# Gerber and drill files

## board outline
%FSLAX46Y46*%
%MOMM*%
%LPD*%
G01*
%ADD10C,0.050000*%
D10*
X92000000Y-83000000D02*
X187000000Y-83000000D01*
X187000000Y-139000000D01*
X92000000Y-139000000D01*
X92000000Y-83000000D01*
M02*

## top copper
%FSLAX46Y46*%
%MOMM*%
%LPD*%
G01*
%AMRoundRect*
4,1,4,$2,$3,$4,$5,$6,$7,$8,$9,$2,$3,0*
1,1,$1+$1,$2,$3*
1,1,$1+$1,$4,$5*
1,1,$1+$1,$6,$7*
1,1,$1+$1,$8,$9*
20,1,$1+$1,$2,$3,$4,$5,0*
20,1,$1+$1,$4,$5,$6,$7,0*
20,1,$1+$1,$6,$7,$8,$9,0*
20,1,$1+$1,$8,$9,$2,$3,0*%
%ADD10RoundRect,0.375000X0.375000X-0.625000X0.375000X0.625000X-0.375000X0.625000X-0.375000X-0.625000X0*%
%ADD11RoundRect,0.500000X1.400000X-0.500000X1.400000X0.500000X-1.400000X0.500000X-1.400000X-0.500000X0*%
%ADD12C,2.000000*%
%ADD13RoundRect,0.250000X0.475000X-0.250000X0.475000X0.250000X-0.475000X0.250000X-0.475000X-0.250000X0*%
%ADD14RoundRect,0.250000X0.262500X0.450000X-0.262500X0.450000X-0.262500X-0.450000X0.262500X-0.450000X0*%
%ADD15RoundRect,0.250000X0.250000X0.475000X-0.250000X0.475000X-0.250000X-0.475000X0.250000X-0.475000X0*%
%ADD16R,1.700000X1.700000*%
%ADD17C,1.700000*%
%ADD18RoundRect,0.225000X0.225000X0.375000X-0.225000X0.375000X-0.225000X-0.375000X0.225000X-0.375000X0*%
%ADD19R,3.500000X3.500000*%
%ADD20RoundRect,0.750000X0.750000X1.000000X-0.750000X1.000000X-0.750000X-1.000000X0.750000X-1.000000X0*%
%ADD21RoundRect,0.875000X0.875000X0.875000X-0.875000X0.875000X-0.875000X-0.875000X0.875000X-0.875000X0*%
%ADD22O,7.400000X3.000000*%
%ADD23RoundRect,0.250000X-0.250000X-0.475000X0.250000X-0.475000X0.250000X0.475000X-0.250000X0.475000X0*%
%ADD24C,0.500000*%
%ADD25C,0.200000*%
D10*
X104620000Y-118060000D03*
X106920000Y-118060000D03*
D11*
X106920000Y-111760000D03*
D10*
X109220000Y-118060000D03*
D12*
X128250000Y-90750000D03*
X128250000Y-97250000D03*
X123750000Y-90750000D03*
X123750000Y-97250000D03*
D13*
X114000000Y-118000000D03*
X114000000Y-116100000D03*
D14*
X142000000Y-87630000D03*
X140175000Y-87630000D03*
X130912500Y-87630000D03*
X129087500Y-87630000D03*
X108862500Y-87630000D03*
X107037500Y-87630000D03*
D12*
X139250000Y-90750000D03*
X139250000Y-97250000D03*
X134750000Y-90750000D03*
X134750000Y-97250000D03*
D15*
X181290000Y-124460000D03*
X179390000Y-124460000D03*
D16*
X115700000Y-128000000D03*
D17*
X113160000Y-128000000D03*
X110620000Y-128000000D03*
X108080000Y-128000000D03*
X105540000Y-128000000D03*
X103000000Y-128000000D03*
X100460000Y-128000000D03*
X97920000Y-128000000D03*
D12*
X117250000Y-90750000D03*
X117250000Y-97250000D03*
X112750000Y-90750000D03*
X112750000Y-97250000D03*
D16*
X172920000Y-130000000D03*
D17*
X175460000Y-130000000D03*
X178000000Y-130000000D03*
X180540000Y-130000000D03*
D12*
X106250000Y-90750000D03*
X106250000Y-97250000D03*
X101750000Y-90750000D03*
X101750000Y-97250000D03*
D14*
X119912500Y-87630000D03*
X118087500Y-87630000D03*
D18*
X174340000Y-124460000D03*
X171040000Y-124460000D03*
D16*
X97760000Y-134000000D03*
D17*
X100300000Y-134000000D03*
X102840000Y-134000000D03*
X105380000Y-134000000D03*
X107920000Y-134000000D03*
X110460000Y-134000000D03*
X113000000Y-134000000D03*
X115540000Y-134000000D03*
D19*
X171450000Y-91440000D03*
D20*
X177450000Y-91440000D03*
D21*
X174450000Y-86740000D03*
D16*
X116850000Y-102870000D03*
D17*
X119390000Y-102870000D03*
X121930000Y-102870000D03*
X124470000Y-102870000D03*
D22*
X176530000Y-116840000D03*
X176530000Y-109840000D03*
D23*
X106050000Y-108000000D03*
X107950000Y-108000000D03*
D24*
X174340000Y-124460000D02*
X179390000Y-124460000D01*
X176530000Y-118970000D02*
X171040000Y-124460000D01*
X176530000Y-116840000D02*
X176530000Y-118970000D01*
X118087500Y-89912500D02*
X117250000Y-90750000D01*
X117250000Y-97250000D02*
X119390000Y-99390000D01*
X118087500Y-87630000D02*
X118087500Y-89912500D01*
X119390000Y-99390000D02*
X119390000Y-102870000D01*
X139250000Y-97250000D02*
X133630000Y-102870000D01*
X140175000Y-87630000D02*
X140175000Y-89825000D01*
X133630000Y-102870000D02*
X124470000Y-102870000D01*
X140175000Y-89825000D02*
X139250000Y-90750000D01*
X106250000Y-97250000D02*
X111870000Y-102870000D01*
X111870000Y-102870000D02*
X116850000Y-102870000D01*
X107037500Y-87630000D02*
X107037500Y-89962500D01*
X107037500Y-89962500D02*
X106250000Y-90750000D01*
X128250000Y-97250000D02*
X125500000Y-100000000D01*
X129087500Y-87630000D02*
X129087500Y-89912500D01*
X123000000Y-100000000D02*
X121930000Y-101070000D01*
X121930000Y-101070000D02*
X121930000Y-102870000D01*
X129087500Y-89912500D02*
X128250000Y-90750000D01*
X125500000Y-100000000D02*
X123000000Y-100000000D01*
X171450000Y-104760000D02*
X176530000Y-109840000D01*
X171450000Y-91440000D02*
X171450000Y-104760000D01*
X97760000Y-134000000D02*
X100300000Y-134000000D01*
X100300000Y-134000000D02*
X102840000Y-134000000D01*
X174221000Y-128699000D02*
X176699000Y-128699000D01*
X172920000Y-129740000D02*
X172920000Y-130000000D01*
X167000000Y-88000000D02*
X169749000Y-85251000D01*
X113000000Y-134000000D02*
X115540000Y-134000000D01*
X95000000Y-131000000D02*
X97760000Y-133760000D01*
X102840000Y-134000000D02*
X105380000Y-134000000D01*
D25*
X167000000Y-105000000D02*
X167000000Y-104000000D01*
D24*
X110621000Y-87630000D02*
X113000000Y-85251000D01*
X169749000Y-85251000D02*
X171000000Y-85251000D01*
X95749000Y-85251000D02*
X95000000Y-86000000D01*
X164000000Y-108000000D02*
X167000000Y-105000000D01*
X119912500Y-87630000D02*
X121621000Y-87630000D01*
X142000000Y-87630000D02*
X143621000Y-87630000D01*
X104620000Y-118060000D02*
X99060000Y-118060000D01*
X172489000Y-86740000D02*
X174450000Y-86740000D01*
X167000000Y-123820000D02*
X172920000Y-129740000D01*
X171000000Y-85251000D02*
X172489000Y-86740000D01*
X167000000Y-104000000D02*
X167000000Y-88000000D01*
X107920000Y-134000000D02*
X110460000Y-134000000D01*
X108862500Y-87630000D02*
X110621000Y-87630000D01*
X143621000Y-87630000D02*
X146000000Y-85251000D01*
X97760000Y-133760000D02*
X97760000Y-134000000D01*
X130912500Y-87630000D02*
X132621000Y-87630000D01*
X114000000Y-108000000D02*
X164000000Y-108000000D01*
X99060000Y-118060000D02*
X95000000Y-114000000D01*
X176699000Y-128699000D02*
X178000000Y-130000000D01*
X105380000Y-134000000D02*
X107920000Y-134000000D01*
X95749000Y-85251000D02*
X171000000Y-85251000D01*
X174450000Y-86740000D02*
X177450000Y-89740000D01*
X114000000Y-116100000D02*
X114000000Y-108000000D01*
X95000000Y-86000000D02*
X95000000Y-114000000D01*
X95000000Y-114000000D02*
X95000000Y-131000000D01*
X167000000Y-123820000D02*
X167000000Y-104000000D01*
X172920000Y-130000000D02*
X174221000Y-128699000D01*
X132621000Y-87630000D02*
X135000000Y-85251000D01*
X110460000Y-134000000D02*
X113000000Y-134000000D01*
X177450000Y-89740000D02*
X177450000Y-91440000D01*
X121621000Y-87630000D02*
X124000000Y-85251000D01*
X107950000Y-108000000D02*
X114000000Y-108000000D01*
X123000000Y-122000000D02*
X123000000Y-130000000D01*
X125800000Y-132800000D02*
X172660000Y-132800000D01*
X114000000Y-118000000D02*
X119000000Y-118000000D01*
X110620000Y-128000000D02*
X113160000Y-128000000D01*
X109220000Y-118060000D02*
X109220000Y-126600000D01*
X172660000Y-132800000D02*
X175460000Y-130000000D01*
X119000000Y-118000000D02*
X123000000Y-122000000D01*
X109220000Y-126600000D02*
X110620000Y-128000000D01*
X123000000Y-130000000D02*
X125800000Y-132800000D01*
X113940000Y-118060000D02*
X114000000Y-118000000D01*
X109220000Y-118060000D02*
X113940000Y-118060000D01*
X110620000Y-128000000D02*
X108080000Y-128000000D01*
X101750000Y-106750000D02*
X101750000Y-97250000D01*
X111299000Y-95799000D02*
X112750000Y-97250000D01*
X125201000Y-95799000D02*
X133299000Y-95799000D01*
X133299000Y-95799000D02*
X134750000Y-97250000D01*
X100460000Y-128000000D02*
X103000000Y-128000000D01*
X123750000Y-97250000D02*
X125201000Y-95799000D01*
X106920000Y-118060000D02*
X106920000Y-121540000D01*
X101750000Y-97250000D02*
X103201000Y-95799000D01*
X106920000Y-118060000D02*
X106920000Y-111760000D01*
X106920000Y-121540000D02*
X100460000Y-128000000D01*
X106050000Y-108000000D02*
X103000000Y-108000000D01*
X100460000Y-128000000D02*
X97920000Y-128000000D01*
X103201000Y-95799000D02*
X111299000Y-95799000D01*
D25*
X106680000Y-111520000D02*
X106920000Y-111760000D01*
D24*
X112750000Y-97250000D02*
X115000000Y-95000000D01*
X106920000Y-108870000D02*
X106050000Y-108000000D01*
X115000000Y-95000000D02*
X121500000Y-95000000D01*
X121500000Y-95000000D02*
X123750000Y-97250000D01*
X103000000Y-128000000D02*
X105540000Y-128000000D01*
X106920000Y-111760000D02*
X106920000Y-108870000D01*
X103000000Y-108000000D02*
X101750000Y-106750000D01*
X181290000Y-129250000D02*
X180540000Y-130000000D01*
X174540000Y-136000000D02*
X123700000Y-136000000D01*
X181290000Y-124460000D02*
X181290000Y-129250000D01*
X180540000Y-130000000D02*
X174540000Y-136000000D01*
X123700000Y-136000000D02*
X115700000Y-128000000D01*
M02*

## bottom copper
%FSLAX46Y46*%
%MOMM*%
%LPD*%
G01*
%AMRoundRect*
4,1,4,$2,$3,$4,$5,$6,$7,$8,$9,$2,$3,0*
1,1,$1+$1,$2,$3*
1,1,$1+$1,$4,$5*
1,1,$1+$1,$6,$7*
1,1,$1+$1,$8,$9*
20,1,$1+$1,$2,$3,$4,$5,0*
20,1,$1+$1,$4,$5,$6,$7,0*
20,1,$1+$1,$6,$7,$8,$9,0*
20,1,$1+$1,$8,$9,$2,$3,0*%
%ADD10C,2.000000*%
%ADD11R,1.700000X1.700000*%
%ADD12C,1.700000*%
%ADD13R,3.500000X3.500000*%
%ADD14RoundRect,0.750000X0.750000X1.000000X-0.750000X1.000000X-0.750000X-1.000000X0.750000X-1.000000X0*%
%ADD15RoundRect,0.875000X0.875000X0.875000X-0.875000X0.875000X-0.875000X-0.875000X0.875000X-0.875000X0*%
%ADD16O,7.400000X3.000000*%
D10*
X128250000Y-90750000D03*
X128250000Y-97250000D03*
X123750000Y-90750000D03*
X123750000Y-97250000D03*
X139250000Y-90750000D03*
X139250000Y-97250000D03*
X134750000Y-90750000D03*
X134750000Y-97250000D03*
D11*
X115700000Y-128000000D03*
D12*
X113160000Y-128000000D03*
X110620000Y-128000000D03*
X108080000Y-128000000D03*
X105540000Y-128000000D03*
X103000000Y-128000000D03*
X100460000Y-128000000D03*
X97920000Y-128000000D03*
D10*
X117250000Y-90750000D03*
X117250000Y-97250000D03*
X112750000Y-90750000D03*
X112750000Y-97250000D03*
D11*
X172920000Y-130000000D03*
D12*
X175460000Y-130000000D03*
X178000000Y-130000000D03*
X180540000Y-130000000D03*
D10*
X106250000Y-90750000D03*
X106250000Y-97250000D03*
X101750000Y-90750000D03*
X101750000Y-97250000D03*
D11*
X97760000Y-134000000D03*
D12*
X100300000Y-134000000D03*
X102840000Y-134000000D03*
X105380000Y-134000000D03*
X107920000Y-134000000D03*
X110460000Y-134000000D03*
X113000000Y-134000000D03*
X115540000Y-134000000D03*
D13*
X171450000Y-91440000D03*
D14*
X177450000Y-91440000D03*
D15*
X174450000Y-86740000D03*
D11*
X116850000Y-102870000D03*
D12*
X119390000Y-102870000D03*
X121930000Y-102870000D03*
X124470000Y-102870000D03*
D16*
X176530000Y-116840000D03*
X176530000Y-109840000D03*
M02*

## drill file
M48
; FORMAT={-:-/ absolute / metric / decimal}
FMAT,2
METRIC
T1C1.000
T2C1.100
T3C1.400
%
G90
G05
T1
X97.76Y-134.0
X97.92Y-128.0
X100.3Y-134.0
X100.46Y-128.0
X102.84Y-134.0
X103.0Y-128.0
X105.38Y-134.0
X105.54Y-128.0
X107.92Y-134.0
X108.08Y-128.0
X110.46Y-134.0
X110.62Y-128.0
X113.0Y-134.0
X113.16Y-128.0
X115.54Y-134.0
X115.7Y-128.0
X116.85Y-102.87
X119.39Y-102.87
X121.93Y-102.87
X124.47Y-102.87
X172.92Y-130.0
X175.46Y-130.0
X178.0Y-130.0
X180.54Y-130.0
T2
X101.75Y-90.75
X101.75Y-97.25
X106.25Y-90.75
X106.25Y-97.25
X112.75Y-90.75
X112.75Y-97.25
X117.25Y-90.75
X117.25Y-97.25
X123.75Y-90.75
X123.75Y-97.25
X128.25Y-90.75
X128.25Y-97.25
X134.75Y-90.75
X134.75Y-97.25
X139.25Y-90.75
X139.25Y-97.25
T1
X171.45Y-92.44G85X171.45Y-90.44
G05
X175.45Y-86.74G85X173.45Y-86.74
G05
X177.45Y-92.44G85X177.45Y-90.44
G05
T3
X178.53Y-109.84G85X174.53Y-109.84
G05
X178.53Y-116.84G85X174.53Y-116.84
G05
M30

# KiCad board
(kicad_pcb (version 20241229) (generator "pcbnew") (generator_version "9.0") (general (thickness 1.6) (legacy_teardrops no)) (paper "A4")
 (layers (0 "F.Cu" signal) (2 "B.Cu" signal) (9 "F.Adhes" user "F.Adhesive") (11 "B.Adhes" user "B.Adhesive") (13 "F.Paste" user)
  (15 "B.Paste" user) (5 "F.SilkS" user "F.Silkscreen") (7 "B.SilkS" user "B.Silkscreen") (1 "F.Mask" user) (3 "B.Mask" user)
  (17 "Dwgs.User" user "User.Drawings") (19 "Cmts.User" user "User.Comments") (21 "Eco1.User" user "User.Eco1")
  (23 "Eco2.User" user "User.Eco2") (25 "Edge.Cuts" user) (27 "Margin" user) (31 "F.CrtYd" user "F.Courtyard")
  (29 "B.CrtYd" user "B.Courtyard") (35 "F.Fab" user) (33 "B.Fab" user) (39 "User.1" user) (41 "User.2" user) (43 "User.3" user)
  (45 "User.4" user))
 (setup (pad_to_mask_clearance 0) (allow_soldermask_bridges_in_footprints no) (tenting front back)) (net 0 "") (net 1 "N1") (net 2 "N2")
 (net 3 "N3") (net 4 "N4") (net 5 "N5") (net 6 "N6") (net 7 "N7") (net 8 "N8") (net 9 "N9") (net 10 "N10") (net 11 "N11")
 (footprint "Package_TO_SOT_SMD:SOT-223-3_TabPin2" (layer "F.Cu") (at 106.92 114.91 90)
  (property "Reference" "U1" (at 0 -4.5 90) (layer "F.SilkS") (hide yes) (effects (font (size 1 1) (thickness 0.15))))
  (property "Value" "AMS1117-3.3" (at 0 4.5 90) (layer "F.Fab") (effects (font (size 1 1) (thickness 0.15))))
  (pad "1" smd roundrect (at -3.15 -2.3 90) (size 2 1.5) (layers "F.Cu" "F.Mask" "F.Paste") (roundrect_rratio 0.25) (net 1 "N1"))
  (pad "2" smd roundrect (at -3.15 0 90) (size 2 1.5) (layers "F.Cu" "F.Mask" "F.Paste") (roundrect_rratio 0.25) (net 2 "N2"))
  (pad "2" smd roundrect (at 3.15 0 90) (size 2 3.8) (layers "F.Cu" "F.Mask" "F.Paste") (roundrect_rratio 0.25) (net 2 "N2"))
  (pad "3" smd roundrect (at -3.15 2.3 90) (size 2 1.5) (layers "F.Cu" "F.Mask" "F.Paste") (roundrect_rratio 0.25) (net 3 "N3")))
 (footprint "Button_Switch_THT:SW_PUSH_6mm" (layer "F.Cu") (at 128.25 90.75 -90)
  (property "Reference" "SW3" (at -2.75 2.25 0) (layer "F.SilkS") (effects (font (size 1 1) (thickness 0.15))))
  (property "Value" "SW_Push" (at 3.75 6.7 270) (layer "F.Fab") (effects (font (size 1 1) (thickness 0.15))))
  (pad "1" thru_hole circle (at 0 0) (size 2 2) (drill 1.1) (layers "*.Cu" "*.Mask") (remove_unused_layers no) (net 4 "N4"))
  (pad "1" thru_hole circle (at 6.5 0) (size 2 2) (drill 1.1) (layers "*.Cu" "*.Mask") (remove_unused_layers no) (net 4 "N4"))
  (pad "2" thru_hole circle (at 0 4.5) (size 2 2) (drill 1.1) (layers "*.Cu" "*.Mask") (remove_unused_layers no) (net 2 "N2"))
  (pad "2" thru_hole circle (at 6.5 4.5) (size 2 2) (drill 1.1) (layers "*.Cu" "*.Mask") (remove_unused_layers no) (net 2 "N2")))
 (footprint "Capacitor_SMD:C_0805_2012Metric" (layer "F.Cu") (at 114 117.05 90)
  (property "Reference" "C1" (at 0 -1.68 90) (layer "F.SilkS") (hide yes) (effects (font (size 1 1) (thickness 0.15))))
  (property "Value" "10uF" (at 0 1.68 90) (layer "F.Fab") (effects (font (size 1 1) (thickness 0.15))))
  (pad "1" smd roundrect (at -0.95 0 90) (size 1 1.45) (layers "F.Cu" "F.Mask" "F.Paste") (roundrect_rratio 0.25) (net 3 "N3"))
  (pad "2" smd roundrect (at 0.95 0 90) (size 1 1.45) (layers "F.Cu" "F.Mask" "F.Paste") (roundrect_rratio 0.25) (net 1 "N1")))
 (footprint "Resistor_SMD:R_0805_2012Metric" (layer "F.Cu") (at 141.0875 87.63 180)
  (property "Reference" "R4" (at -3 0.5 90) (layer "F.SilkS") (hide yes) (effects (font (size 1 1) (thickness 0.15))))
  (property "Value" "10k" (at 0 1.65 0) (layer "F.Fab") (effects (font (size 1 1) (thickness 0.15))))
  (pad "1" smd roundrect (at -0.9125 0 180) (size 1.025 1.4) (layers "F.Cu" "F.Mask" "F.Paste") (roundrect_rratio 0.243902) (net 1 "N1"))
  (pad "2" smd roundrect (at 0.9125 0 180) (size 1.025 1.4) (layers "F.Cu" "F.Mask" "F.Paste") (roundrect_rratio 0.243902) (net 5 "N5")))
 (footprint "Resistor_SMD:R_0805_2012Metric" (layer "F.Cu") (at 130 87.63 180)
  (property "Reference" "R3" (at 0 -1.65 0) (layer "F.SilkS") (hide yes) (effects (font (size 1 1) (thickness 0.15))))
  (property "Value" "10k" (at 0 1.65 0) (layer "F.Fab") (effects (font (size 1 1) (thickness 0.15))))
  (pad "1" smd roundrect (at -0.9125 0 180) (size 1.025 1.4) (layers "F.Cu" "F.Mask" "F.Paste") (roundrect_rratio 0.243902) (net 1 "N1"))
  (pad "2" smd roundrect (at 0.9125 0 180) (size 1.025 1.4) (layers "F.Cu" "F.Mask" "F.Paste") (roundrect_rratio 0.243902) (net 4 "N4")))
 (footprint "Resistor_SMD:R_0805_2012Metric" (layer "F.Cu") (at 107.95 87.63 180)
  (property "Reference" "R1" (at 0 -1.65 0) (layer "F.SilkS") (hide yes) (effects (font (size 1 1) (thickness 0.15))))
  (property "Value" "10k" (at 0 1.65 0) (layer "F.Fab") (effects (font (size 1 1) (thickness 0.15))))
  (pad "1" smd roundrect (at -0.9125 0 180) (size 1.025 1.4) (layers "F.Cu" "F.Mask" "F.Paste") (roundrect_rratio 0.243902) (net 1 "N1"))
  (pad "2" smd roundrect (at 0.9125 0 180) (size 1.025 1.4) (layers "F.Cu" "F.Mask" "F.Paste") (roundrect_rratio 0.243902) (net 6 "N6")))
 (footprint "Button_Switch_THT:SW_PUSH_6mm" (layer "F.Cu") (at 139.25 90.75 -90)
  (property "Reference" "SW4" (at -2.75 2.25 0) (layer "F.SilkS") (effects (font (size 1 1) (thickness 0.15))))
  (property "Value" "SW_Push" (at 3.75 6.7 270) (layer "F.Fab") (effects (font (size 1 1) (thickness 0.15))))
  (pad "1" thru_hole circle (at 0 0) (size 2 2) (drill 1.1) (layers "*.Cu" "*.Mask") (remove_unused_layers no) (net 5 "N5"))
  (pad "1" thru_hole circle (at 6.5 0) (size 2 2) (drill 1.1) (layers "*.Cu" "*.Mask") (remove_unused_layers no) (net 5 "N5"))
  (pad "2" thru_hole circle (at 0 4.5) (size 2 2) (drill 1.1) (layers "*.Cu" "*.Mask") (remove_unused_layers no) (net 2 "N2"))
  (pad "2" thru_hole circle (at 6.5 4.5) (size 2 2) (drill 1.1) (layers "*.Cu" "*.Mask") (remove_unused_layers no) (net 2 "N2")))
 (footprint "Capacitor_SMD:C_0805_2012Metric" (layer "F.Cu") (at 180.34 124.46 180)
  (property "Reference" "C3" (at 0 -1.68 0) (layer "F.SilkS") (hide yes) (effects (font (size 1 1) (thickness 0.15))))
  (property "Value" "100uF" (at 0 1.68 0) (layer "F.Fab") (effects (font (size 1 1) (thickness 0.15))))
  (pad "1" smd roundrect (at -0.95 0 180) (size 1 1.45) (layers "F.Cu" "F.Mask" "F.Paste") (roundrect_rratio 0.25) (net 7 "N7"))
  (pad "2" smd roundrect (at 0.95 0 180) (size 1 1.45) (layers "F.Cu" "F.Mask" "F.Paste") (roundrect_rratio 0.25) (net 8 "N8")))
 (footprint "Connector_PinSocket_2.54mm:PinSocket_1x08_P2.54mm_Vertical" (layer "F.Cu") (at 115.7 128 -90)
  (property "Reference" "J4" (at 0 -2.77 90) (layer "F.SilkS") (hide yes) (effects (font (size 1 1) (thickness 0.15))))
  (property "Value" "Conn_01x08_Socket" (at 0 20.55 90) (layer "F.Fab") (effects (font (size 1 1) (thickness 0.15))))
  (pad "1" thru_hole rect (at 0 0 270) (size 1.7 1.7) (drill 1) (layers "*.Cu" "*.Mask") (remove_unused_layers no) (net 7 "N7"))
  (pad "2" thru_hole circle (at 0 2.54 270) (size 1.7 1.7) (drill 1) (layers "*.Cu" "*.Mask") (remove_unused_layers no) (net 3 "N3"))
  (pad "3" thru_hole circle (at 0 5.08 270) (size 1.7 1.7) (drill 1) (layers "*.Cu" "*.Mask") (remove_unused_layers no) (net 3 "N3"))
  (pad "4" thru_hole circle (at 0 7.62 270) (size 1.7 1.7) (drill 1) (layers "*.Cu" "*.Mask") (remove_unused_layers no) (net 3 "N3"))
  (pad "5" thru_hole circle (at 0 10.16 270) (size 1.7 1.7) (drill 1) (layers "*.Cu" "*.Mask") (remove_unused_layers no) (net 2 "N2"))
  (pad "6" thru_hole circle (at 0 12.7 270) (size 1.7 1.7) (drill 1) (layers "*.Cu" "*.Mask") (remove_unused_layers no) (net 2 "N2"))
  (pad "7" thru_hole circle (at 0 15.24 270) (size 1.7 1.7) (drill 1) (layers "*.Cu" "*.Mask") (remove_unused_layers no) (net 2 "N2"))
  (pad "8" thru_hole circle (at 0 17.78 270) (size 1.7 1.7) (drill 1) (layers "*.Cu" "*.Mask") (remove_unused_layers no) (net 2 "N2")))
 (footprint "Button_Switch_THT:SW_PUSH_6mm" (layer "F.Cu") (at 117.25 90.75 -90)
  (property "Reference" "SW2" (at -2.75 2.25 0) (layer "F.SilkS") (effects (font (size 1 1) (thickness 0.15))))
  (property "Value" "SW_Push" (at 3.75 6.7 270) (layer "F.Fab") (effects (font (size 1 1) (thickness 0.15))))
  (pad "1" thru_hole circle (at 0 0) (size 2 2) (drill 1.1) (layers "*.Cu" "*.Mask") (remove_unused_layers no) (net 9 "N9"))
  (pad "1" thru_hole circle (at 6.5 0) (size 2 2) (drill 1.1) (layers "*.Cu" "*.Mask") (remove_unused_layers no) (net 9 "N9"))
  (pad "2" thru_hole circle (at 0 4.5) (size 2 2) (drill 1.1) (layers "*.Cu" "*.Mask") (remove_unused_layers no) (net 2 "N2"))
  (pad "2" thru_hole circle (at 6.5 4.5) (size 2 2) (drill 1.1) (layers "*.Cu" "*.Mask") (remove_unused_layers no) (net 2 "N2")))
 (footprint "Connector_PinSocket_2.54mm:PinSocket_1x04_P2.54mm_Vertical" (layer "F.Cu") (at 172.92 130 90)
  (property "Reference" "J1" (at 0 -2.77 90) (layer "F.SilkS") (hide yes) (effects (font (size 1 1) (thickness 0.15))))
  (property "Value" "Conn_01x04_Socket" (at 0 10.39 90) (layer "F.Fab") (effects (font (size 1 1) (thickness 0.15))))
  (pad "1" thru_hole rect (at 0 0 90) (size 1.7 1.7) (drill 1) (layers "*.Cu" "*.Mask") (remove_unused_layers no) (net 1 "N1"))
  (pad "2" thru_hole circle (at 0 2.54 90) (size 1.7 1.7) (drill 1) (layers "*.Cu" "*.Mask") (remove_unused_layers no) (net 3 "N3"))
  (pad "3" thru_hole circle (at 0 5.08 90) (size 1.7 1.7) (drill 1) (layers "*.Cu" "*.Mask") (remove_unused_layers no) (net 1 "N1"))
  (pad "4" thru_hole circle (at 0 7.62 90) (size 1.7 1.7) (drill 1) (layers "*.Cu" "*.Mask") (remove_unused_layers no) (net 7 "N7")))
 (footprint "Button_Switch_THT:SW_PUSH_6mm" (layer "F.Cu") (at 106.25 90.75 -90)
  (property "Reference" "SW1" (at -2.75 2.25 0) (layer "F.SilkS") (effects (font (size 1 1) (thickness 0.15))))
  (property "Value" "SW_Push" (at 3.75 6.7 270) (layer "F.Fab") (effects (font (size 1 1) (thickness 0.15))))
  (pad "1" thru_hole circle (at 0 0) (size 2 2) (drill 1.1) (layers "*.Cu" "*.Mask") (remove_unused_layers no) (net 6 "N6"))
  (pad "1" thru_hole circle (at 6.5 0) (size 2 2) (drill 1.1) (layers "*.Cu" "*.Mask") (remove_unused_layers no) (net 6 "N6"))
  (pad "2" thru_hole circle (at 0 4.5) (size 2 2) (drill 1.1) (layers "*.Cu" "*.Mask") (remove_unused_layers no) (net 2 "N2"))
  (pad "2" thru_hole circle (at 6.5 4.5) (size 2 2) (drill 1.1) (layers "*.Cu" "*.Mask") (remove_unused_layers no) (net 2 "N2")))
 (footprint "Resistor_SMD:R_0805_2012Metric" (layer "F.Cu") (at 119 87.63 180)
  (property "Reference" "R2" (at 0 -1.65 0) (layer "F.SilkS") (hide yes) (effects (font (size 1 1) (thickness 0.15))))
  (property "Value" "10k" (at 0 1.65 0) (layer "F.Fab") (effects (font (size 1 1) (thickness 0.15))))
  (pad "1" smd roundrect (at -0.9125 0 180) (size 1.025 1.4) (layers "F.Cu" "F.Mask" "F.Paste") (roundrect_rratio 0.243902) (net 1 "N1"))
  (pad "2" smd roundrect (at 0.9125 0 180) (size 1.025 1.4) (layers "F.Cu" "F.Mask" "F.Paste") (roundrect_rratio 0.243902) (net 9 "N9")))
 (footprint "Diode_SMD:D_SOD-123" (layer "F.Cu") (at 172.69 124.46 180)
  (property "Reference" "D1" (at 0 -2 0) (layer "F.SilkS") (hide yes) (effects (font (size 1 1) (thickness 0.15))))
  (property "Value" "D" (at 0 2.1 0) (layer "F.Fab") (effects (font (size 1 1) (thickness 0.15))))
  (pad "1" smd roundrect (at -1.65 0 180) (size 0.9 1.2) (layers "F.Cu" "F.Mask" "F.Paste") (roundrect_rratio 0.25) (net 8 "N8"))
  (pad "2" smd roundrect (at 1.65 0 180) (size 0.9 1.2) (layers "F.Cu" "F.Mask" "F.Paste") (roundrect_rratio 0.25) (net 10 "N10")))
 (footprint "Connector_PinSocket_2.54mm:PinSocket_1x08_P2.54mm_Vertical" (layer "F.Cu") (at 97.76 134 90)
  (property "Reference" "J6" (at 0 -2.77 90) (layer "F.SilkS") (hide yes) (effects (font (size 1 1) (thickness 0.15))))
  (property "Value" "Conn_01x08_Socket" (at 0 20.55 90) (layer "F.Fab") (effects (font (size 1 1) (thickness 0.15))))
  (pad "1" thru_hole rect (at 0 0 90) (size 1.7 1.7) (drill 1) (layers "*.Cu" "*.Mask") (remove_unused_layers no) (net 1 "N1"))
  (pad "2" thru_hole circle (at 0 2.54 90) (size 1.7 1.7) (drill 1) (layers "*.Cu" "*.Mask") (remove_unused_layers no) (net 1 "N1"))
  (pad "3" thru_hole circle (at 0 5.08 90) (size 1.7 1.7) (drill 1) (layers "*.Cu" "*.Mask") (remove_unused_layers no) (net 1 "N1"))
  (pad "4" thru_hole circle (at 0 7.62 90) (size 1.7 1.7) (drill 1) (layers "*.Cu" "*.Mask") (remove_unused_layers no) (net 1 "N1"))
  (pad "5" thru_hole circle (at 0 10.16 90) (size 1.7 1.7) (drill 1) (layers "*.Cu" "*.Mask") (remove_unused_layers no) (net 1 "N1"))
  (pad "6" thru_hole circle (at 0 12.7 90) (size 1.7 1.7) (drill 1) (layers "*.Cu" "*.Mask") (remove_unused_layers no) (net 1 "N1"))
  (pad "7" thru_hole circle (at 0 15.24 90) (size 1.7 1.7) (drill 1) (layers "*.Cu" "*.Mask") (remove_unused_layers no) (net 1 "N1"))
  (pad "8" thru_hole circle (at 0 17.78 90) (size 1.7 1.7) (drill 1) (layers "*.Cu" "*.Mask") (remove_unused_layers no) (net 1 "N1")))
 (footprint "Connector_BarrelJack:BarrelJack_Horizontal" (layer "F.Cu") (at 171.45 91.44 180)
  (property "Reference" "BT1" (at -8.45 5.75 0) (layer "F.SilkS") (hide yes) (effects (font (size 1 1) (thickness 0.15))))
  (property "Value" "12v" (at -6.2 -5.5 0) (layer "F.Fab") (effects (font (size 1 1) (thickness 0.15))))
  (pad "1" thru_hole rect (at 0 0 180) (size 3.5 3.5) (drill oval 1 3) (layers "*.Cu" "*.Mask") (remove_unused_layers no) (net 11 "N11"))
  (pad "2" thru_hole roundrect (at -6 0 180) (size 3 3.5) (drill oval 1 3) (layers "*.Cu" "*.Mask") (remove_unused_layers no)
   (roundrect_rratio 0.25) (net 1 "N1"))
  (pad "3" thru_hole roundrect (at -3 4.7 180) (size 3.5 3.5) (drill oval 3 1) (layers "*.Cu" "*.Mask") (remove_unused_layers no)
   (roundrect_rratio 0.25) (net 1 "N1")))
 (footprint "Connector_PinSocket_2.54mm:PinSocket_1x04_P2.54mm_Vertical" (layer "F.Cu") (at 116.85 102.87 90)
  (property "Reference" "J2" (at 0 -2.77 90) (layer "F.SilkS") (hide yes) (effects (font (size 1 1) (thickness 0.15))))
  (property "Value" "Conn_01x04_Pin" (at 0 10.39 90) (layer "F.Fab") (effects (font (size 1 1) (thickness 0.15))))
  (pad "1" thru_hole rect (at 0 0 90) (size 1.7 1.7) (drill 1) (layers "*.Cu" "*.Mask") (remove_unused_layers no) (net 6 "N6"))
  (pad "2" thru_hole circle (at 0 2.54 90) (size 1.7 1.7) (drill 1) (layers "*.Cu" "*.Mask") (remove_unused_layers no) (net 9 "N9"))
  (pad "3" thru_hole circle (at 0 5.08 90) (size 1.7 1.7) (drill 1) (layers "*.Cu" "*.Mask") (remove_unused_layers no) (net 4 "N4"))
  (pad "4" thru_hole circle (at 0 7.62 90) (size 1.7 1.7) (drill 1) (layers "*.Cu" "*.Mask") (remove_unused_layers no) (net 5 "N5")))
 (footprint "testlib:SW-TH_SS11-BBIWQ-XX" (layer "F.Cu") (at 176.53 113.34 90)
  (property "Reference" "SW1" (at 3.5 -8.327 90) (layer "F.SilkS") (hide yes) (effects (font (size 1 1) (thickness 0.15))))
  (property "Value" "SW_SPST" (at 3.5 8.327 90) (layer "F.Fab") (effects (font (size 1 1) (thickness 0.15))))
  (pad "1" thru_hole oval (at -3.5 0 270) (size 3 7.4) (drill oval 1.4 5.4) (layers "*.Cu" "*.Mask") (remove_unused_layers no)
   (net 10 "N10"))
  (pad "2" thru_hole oval (at 3.5 0 270) (size 3 7.4) (drill oval 1.4 5.4) (layers "*.Cu" "*.Mask") (remove_unused_layers no) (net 11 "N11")))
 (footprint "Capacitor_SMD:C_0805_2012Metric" (layer "F.Cu") (at 107 108)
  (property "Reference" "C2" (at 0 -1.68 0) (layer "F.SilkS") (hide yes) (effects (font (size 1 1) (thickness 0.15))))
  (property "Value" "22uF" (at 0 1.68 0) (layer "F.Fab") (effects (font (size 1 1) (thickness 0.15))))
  (pad "1" smd roundrect (at -0.95 0) (size 1 1.45) (layers "F.Cu" "F.Mask" "F.Paste") (roundrect_rratio 0.25) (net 2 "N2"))
  (pad "2" smd roundrect (at 0.95 0) (size 1 1.45) (layers "F.Cu" "F.Mask" "F.Paste") (roundrect_rratio 0.25) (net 1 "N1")))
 (gr_rect (start 92 83) (end 187 139) (stroke (width 0.05) (type default)) (fill no) (layer "Edge.Cuts"))
 (segment (start 174.34 124.46) (end 179.39 124.46) (width 0.5) (layer "F.Cu") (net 8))
 (segment (start 176.53 118.97) (end 171.04 124.46) (width 0.5) (layer "F.Cu") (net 10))
 (segment (start 176.53 116.84) (end 176.53 118.97) (width 0.5) (layer "F.Cu") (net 10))
 (segment (start 118.0875 89.9125) (end 117.25 90.75) (width 0.5) (layer "F.Cu") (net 9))
 (segment (start 117.25 97.25) (end 119.39 99.39) (width 0.5) (layer "F.Cu") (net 9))
 (segment (start 118.0875 87.63) (end 118.0875 89.9125) (width 0.5) (layer "F.Cu") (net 9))
 (segment (start 119.39 99.39) (end 119.39 102.87) (width 0.5) (layer "F.Cu") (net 9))
 (segment (start 139.25 97.25) (end 133.63 102.87) (width 0.5) (layer "F.Cu") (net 5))
 (segment (start 140.175 87.63) (end 140.175 89.825) (width 0.5) (layer "F.Cu") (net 5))
 (segment (start 133.63 102.87) (end 124.47 102.87) (width 0.5) (layer "F.Cu") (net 5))
 (segment (start 140.175 89.825) (end 139.25 90.75) (width 0.5) (layer "F.Cu") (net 5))
 (segment (start 106.25 97.25) (end 111.87 102.87) (width 0.5) (layer "F.Cu") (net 6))
 (segment (start 111.87 102.87) (end 116.85 102.87) (width 0.5) (layer "F.Cu") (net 6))
 (segment (start 107.0375 87.63) (end 107.0375 89.9625) (width 0.5) (layer "F.Cu") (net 6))
 (segment (start 107.0375 89.9625) (end 106.25 90.75) (width 0.5) (layer "F.Cu") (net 6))
 (segment (start 128.25 97.25) (end 125.5 100) (width 0.5) (layer "F.Cu") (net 4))
 (segment (start 129.0875 87.63) (end 129.0875 89.9125) (width 0.5) (layer "F.Cu") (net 4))
 (segment (start 123 100) (end 121.93 101.07) (width 0.5) (layer "F.Cu") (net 4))
 (segment (start 121.93 101.07) (end 121.93 102.87) (width 0.5) (layer "F.Cu") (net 4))
 (segment (start 129.0875 89.9125) (end 128.25 90.75) (width 0.5) (layer "F.Cu") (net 4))
 (segment (start 125.5 100) (end 123 100) (width 0.5) (layer "F.Cu") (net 4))
 (segment (start 171.45 104.76) (end 176.53 109.84) (width 0.5) (layer "F.Cu") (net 11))
 (segment (start 171.45 91.44) (end 171.45 104.76) (width 0.5) (layer "F.Cu") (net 11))
 (segment (start 97.76 134) (end 100.3 134) (width 0.5) (layer "F.Cu") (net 1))
 (segment (start 100.3 134) (end 102.84 134) (width 0.5) (layer "F.Cu") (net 1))
 (segment (start 174.221 128.699) (end 176.699 128.699) (width 0.5) (layer "F.Cu") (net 1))
 (segment (start 172.92 129.74) (end 172.92 130) (width 0.5) (layer "F.Cu") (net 1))
 (segment (start 167 88) (end 169.749 85.251) (width 0.5) (layer "F.Cu") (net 1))
 (segment (start 113 134) (end 115.54 134) (width 0.5) (layer "F.Cu") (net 1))
 (segment (start 95 131) (end 97.76 133.76) (width 0.5) (layer "F.Cu") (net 1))
 (segment (start 102.84 134) (end 105.38 134) (width 0.5) (layer "F.Cu") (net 1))
 (segment (start 167 105) (end 167 104) (width 0.2) (layer "F.Cu") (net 1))
 (segment (start 110.621 87.63) (end 113 85.251) (width 0.5) (layer "F.Cu") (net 1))
 (segment (start 169.749 85.251) (end 171 85.251) (width 0.5) (layer "F.Cu") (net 1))
 (segment (start 95.749 85.251) (end 95 86) (width 0.5) (layer "F.Cu") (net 1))
 (segment (start 164 108) (end 167 105) (width 0.5) (layer "F.Cu") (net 1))
 (segment (start 119.9125 87.63) (end 121.621 87.63) (width 0.5) (layer "F.Cu") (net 1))
 (segment (start 142 87.63) (end 143.621 87.63) (width 0.5) (layer "F.Cu") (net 1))
 (segment (start 104.62 118.06) (end 99.06 118.06) (width 0.5) (layer "F.Cu") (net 1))
 (segment (start 172.489 86.74) (end 174.45 86.74) (width 0.5) (layer "F.Cu") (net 1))
 (segment (start 167 123.82) (end 172.92 129.74) (width 0.5) (layer "F.Cu") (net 1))
 (segment (start 171 85.251) (end 172.489 86.74) (width 0.5) (layer "F.Cu") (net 1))
 (segment (start 167 104) (end 167 88) (width 0.5) (layer "F.Cu") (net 1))
 (segment (start 107.92 134) (end 110.46 134) (width 0.5) (layer "F.Cu") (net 1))
 (segment (start 108.8625 87.63) (end 110.621 87.63) (width 0.5) (layer "F.Cu") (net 1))
 (segment (start 143.621 87.63) (end 146 85.251) (width 0.5) (layer "F.Cu") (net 1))
 (segment (start 97.76 133.76) (end 97.76 134) (width 0.5) (layer "F.Cu") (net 1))
 (segment (start 130.9125 87.63) (end 132.621 87.63) (width 0.5) (layer "F.Cu") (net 1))
 (segment (start 114 108) (end 164 108) (width 0.5) (layer "F.Cu") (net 1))
 (segment (start 99.06 118.06) (end 95 114) (width 0.5) (layer "F.Cu") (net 1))
 (segment (start 176.699 128.699) (end 178 130) (width 0.5) (layer "F.Cu") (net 1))
 (segment (start 105.38 134) (end 107.92 134) (width 0.5) (layer "F.Cu") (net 1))
 (segment (start 95.749 85.251) (end 171 85.251) (width 0.5) (layer "F.Cu") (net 1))
 (segment (start 174.45 86.74) (end 177.45 89.74) (width 0.5) (layer "F.Cu") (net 1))
 (segment (start 114 116.1) (end 114 108) (width 0.5) (layer "F.Cu") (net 1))
 (segment (start 95 86) (end 95 114) (width 0.5) (layer "F.Cu") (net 1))
 (segment (start 95 114) (end 95 131) (width 0.5) (layer "F.Cu") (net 1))
 (segment (start 167 123.82) (end 167 104) (width 0.5) (layer "F.Cu") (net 1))
 (segment (start 172.92 130) (end 174.221 128.699) (width 0.5) (layer "F.Cu") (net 1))
 (segment (start 132.621 87.63) (end 135 85.251) (width 0.5) (layer "F.Cu") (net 1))
 (segment (start 110.46 134) (end 113 134) (width 0.5) (layer "F.Cu") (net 1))
 (segment (start 177.45 89.74) (end 177.45 91.44) (width 0.5) (layer "F.Cu") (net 1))
 (segment (start 121.621 87.63) (end 124 85.251) (width 0.5) (layer "F.Cu") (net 1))
 (segment (start 107.95 108) (end 114 108) (width 0.5) (layer "F.Cu") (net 1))
 (segment (start 123 122) (end 123 130) (width 0.5) (layer "F.Cu") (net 3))
 (segment (start 125.8 132.8) (end 172.66 132.8) (width 0.5) (layer "F.Cu") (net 3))
 (segment (start 114 118) (end 119 118) (width 0.5) (layer "F.Cu") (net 3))
 (segment (start 110.62 128) (end 113.16 128) (width 0.5) (layer "F.Cu") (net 3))
 (segment (start 109.22 118.06) (end 109.22 126.6) (width 0.5) (layer "F.Cu") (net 3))
 (segment (start 172.66 132.8) (end 175.46 130) (width 0.5) (layer "F.Cu") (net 3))
 (segment (start 119 118) (end 123 122) (width 0.5) (layer "F.Cu") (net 3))
 (segment (start 109.22 126.6) (end 110.62 128) (width 0.5) (layer "F.Cu") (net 3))
 (segment (start 123 130) (end 125.8 132.8) (width 0.5) (layer "F.Cu") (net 3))
 (segment (start 113.94 118.06) (end 114 118) (width 0.5) (layer "F.Cu") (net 3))
 (segment (start 109.22 118.06) (end 113.94 118.06) (width 0.5) (layer "F.Cu") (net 3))
 (segment (start 110.62 128) (end 108.08 128) (width 0.5) (layer "F.Cu") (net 3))
 (segment (start 101.75 106.75) (end 101.75 97.25) (width 0.5) (layer "F.Cu") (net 2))
 (segment (start 111.299 95.799) (end 112.75 97.25) (width 0.5) (layer "F.Cu") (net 2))
 (segment (start 125.201 95.799) (end 133.299 95.799) (width 0.5) (layer "F.Cu") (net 2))
 (segment (start 133.299 95.799) (end 134.75 97.25) (width 0.5) (layer "F.Cu") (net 2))
 (segment (start 100.46 128) (end 103 128) (width 0.5) (layer "F.Cu") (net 2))
 (segment (start 123.75 97.25) (end 125.201 95.799) (width 0.5) (layer "F.Cu") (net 2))
 (segment (start 106.92 118.06) (end 106.92 121.54) (width 0.5) (layer "F.Cu") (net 2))
 (segment (start 101.75 97.25) (end 103.201 95.799) (width 0.5) (layer "F.Cu") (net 2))
 (segment (start 106.92 118.06) (end 106.92 111.76) (width 0.5) (layer "F.Cu") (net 2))
 (segment (start 106.92 121.54) (end 100.46 128) (width 0.5) (layer "F.Cu") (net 2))
 (segment (start 106.05 108) (end 103 108) (width 0.5) (layer "F.Cu") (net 2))
 (segment (start 100.46 128) (end 97.92 128) (width 0.5) (layer "F.Cu") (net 2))
 (segment (start 103.201 95.799) (end 111.299 95.799) (width 0.5) (layer "F.Cu") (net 2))
 (segment (start 106.68 111.52) (end 106.92 111.76) (width 0.2) (layer "F.Cu") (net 2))
 (segment (start 112.75 97.25) (end 115 95) (width 0.5) (layer "F.Cu") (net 2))
 (segment (start 106.92 108.87) (end 106.05 108) (width 0.5) (layer "F.Cu") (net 2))
 (segment (start 115 95) (end 121.5 95) (width 0.5) (layer "F.Cu") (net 2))
 (segment (start 121.5 95) (end 123.75 97.25) (width 0.5) (layer "F.Cu") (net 2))
 (segment (start 103 128) (end 105.54 128) (width 0.5) (layer "F.Cu") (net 2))
 (segment (start 106.92 111.76) (end 106.92 108.87) (width 0.5) (layer "F.Cu") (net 2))
 (segment (start 103 108) (end 101.75 106.75) (width 0.5) (layer "F.Cu") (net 2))
 (segment (start 181.29 129.25) (end 180.54 130) (width 0.5) (layer "F.Cu") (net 7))
 (segment (start 174.54 136) (end 123.7 136) (width 0.5) (layer "F.Cu") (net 7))
 (segment (start 181.29 124.46) (end 181.29 129.25) (width 0.5) (layer "F.Cu") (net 7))
 (segment (start 180.54 130) (end 174.54 136) (width 0.5) (layer "F.Cu") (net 7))
 (segment (start 123.7 136) (end 115.7 128) (width 0.5) (layer "F.Cu") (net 7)))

